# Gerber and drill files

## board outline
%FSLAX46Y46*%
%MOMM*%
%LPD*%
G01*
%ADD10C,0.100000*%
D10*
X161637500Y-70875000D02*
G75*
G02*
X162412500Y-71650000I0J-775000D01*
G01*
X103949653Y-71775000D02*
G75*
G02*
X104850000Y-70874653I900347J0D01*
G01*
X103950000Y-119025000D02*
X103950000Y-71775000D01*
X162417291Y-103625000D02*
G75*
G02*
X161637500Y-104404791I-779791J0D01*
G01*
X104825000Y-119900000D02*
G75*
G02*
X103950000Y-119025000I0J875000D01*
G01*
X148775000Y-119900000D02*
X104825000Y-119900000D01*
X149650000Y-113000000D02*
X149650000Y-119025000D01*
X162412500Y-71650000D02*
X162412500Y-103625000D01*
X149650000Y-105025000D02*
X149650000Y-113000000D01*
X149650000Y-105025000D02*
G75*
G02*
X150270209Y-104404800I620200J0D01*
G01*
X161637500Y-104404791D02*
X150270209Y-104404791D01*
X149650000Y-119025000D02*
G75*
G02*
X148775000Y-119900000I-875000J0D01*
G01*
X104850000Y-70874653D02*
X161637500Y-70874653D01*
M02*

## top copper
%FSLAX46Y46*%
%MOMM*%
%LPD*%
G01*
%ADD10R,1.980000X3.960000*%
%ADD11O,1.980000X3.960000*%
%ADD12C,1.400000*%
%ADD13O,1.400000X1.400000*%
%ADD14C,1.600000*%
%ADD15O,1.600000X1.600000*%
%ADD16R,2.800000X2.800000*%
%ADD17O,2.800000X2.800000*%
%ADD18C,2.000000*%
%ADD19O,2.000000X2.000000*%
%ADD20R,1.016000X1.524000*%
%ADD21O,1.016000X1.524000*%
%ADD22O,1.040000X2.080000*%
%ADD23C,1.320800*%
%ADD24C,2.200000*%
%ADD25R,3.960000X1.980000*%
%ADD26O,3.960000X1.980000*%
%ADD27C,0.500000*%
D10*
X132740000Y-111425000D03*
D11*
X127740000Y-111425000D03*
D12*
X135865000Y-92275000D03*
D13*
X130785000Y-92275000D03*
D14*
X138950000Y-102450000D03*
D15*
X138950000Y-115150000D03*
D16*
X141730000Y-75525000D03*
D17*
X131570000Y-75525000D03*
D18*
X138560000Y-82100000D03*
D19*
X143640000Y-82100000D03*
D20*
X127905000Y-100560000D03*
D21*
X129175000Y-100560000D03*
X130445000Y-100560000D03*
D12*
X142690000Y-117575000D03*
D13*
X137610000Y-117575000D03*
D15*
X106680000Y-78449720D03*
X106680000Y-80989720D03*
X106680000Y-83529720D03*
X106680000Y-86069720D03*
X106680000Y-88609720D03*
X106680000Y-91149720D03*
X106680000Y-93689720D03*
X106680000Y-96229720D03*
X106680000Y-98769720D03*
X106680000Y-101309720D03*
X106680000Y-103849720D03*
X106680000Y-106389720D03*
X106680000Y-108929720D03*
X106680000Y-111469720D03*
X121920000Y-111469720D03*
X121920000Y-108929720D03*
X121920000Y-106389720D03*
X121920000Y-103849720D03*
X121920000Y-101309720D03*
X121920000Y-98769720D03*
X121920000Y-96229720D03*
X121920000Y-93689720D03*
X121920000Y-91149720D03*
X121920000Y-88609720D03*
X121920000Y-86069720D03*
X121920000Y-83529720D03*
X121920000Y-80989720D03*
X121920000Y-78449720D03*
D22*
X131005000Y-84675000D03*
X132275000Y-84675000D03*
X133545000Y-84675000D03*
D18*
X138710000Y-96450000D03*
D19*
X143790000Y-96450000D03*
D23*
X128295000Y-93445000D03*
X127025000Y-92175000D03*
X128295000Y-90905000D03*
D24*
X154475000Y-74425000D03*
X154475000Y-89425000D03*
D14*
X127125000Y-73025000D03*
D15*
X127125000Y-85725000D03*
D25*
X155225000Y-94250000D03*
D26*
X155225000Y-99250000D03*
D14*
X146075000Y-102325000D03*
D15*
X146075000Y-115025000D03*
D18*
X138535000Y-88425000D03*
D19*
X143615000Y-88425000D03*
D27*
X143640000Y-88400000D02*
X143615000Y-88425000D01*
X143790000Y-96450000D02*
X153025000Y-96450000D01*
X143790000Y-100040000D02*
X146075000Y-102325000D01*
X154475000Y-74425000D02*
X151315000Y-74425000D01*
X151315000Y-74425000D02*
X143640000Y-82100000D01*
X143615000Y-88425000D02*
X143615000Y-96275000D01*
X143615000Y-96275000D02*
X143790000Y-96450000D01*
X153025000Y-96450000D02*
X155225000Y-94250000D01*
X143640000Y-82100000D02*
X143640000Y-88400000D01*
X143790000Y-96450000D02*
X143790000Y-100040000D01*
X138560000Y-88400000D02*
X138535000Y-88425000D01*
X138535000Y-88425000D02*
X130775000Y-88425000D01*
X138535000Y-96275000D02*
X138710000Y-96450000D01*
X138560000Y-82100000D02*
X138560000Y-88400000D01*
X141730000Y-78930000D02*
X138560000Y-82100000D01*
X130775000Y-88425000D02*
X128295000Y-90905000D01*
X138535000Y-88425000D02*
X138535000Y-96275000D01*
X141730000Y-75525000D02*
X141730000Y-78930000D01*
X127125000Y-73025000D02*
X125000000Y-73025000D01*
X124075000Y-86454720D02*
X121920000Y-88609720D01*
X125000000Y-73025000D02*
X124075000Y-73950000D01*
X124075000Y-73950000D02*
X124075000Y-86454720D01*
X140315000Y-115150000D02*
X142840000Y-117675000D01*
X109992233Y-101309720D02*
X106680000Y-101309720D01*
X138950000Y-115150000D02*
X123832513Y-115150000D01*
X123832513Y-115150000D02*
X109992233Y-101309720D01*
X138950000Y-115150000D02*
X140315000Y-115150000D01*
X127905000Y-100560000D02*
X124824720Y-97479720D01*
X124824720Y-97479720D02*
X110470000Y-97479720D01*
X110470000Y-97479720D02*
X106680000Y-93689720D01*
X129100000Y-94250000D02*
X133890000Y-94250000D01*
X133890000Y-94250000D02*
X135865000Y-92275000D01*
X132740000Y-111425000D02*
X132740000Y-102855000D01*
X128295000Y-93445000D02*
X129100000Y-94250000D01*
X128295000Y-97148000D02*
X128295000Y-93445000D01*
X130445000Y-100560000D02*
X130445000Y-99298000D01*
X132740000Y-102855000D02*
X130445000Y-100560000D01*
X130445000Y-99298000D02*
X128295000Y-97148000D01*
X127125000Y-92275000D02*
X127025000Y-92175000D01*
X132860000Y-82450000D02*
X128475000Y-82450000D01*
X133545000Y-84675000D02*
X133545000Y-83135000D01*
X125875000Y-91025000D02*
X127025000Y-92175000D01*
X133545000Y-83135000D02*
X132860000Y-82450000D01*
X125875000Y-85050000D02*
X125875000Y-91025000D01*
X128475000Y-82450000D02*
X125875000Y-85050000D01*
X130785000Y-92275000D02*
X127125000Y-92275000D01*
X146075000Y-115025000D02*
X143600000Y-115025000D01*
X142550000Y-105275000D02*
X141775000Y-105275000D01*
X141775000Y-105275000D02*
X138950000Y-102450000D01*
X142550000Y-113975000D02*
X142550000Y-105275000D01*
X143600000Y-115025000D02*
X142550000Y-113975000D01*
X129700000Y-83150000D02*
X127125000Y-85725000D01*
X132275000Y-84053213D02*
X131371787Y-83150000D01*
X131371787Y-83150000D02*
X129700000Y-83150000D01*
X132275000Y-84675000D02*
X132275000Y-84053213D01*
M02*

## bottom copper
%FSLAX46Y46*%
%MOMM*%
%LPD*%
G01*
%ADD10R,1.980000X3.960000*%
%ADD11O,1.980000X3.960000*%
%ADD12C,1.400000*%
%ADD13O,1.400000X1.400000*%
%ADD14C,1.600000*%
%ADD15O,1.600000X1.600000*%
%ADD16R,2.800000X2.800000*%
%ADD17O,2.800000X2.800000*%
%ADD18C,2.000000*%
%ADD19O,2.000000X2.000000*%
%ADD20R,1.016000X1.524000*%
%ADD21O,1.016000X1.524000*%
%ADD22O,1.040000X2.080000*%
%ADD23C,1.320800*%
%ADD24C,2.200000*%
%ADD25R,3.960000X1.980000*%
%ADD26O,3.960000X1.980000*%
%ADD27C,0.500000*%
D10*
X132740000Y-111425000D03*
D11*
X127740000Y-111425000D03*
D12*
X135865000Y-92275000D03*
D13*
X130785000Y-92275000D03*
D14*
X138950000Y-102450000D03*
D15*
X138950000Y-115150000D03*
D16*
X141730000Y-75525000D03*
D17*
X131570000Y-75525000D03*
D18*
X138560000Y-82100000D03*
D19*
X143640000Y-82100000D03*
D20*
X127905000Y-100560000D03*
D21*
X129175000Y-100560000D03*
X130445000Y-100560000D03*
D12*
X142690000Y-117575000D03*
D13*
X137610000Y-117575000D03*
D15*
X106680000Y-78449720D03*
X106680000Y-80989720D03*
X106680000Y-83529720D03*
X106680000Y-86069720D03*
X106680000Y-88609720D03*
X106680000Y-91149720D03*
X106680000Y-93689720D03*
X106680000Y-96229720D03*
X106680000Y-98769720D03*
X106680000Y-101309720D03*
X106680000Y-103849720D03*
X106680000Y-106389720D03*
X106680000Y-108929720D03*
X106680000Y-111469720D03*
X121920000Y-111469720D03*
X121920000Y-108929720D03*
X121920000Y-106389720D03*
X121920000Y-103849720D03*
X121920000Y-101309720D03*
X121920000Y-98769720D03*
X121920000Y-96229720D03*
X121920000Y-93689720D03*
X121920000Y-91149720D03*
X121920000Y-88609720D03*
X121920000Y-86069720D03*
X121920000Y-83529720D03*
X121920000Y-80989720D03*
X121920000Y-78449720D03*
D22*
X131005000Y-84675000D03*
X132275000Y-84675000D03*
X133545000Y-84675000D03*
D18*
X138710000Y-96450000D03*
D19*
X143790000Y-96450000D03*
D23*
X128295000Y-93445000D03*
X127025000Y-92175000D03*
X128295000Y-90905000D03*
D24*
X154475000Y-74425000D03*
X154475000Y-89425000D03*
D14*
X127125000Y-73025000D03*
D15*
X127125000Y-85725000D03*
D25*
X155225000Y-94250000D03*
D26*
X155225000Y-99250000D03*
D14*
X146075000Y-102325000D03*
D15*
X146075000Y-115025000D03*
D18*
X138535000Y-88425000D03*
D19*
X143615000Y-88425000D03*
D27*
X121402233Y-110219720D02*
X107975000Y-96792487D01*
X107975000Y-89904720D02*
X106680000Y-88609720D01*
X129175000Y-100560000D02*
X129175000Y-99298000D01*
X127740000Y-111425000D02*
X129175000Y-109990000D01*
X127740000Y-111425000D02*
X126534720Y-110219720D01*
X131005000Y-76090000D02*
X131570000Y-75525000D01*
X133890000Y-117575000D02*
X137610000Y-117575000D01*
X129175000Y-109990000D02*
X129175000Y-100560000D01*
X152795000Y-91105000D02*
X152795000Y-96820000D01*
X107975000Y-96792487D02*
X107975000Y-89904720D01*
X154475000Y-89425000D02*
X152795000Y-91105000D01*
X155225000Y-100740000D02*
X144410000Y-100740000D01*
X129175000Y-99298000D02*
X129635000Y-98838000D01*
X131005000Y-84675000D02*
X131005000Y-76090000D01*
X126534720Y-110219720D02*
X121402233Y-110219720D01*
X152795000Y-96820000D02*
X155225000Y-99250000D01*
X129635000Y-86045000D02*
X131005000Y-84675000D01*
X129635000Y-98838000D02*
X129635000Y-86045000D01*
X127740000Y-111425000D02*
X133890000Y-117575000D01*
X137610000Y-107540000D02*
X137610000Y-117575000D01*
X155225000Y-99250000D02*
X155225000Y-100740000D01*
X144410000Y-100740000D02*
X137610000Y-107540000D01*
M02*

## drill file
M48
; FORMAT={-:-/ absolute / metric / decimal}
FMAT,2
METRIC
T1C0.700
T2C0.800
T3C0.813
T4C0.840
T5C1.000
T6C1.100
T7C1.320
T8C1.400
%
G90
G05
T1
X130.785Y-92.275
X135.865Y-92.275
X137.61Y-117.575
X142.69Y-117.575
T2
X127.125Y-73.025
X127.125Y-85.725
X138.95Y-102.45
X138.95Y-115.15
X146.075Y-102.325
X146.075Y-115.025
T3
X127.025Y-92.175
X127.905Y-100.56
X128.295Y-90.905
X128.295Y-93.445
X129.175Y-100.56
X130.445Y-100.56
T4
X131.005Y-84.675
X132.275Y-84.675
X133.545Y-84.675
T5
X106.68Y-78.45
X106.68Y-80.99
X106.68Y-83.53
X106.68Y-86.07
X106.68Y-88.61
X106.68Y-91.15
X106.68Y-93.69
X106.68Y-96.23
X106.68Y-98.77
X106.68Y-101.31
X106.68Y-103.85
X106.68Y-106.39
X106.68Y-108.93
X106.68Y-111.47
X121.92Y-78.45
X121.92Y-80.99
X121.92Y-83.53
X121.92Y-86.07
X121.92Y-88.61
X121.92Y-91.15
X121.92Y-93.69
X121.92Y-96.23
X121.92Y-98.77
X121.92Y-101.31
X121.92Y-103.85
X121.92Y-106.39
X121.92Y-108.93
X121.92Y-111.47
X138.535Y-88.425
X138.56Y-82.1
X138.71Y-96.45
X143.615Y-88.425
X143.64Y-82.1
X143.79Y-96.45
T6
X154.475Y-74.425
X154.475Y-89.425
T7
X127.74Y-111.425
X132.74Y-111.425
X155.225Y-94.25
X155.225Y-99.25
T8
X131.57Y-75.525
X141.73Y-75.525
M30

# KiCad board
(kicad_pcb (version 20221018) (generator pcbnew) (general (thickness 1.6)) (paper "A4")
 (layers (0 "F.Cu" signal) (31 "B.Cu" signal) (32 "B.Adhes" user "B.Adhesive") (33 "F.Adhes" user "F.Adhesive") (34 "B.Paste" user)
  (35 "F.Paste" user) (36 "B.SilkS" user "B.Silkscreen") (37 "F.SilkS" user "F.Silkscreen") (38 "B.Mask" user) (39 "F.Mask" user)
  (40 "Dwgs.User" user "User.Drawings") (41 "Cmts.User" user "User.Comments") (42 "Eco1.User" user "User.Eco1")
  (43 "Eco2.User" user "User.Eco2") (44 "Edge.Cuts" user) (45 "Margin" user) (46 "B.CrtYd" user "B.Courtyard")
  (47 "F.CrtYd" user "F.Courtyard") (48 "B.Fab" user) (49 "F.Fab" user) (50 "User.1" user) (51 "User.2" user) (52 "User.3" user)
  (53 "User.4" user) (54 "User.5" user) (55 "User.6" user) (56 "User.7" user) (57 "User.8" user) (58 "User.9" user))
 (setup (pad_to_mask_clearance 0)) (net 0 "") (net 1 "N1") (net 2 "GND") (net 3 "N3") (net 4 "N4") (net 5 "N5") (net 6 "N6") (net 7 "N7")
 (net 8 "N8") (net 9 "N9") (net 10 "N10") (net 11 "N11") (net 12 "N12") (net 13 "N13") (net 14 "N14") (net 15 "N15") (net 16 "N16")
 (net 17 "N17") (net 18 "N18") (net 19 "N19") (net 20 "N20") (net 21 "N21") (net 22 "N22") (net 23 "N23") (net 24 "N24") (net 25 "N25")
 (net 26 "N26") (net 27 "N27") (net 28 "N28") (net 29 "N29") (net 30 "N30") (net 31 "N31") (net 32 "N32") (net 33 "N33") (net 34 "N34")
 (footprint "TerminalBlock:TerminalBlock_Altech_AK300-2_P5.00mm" (layer "F.Cu") (at 132.74 111.425 180)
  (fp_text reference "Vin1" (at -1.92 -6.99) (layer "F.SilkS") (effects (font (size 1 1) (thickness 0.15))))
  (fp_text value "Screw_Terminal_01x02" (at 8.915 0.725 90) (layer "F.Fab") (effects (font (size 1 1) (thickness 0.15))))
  (pad "1" thru_hole rect (at 0 0 180) (size 1.98 3.96) (drill 1.32) (layers "*.Cu" "*.Mask") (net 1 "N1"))
  (pad "2" thru_hole oval (at 5 0 180) (size 1.98 3.96) (drill 1.32) (layers "*.Cu" "*.Mask") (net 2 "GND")))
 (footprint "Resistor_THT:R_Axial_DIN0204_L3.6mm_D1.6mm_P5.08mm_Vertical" (layer "F.Cu") (at 135.865 92.275 180)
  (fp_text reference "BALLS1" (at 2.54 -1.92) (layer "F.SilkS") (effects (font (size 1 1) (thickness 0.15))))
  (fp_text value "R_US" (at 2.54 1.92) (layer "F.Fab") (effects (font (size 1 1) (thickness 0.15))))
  (pad "1" thru_hole circle (at 0 0 180) (size 1.4 1.4) (drill 0.7) (layers "*.Cu" "*.Mask") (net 1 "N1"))
  (pad "2" thru_hole oval (at 5.08 0 180) (size 1.4 1.4) (drill 0.7) (layers "*.Cu" "*.Mask") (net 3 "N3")))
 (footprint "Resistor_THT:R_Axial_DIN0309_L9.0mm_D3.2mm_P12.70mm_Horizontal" (layer "F.Cu") (at 138.95 102.45 -90)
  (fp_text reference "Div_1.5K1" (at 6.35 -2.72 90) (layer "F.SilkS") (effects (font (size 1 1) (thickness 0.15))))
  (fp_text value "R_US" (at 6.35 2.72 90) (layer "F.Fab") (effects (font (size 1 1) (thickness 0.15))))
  (pad "1" thru_hole circle (at 0 0 270) (size 1.6 1.6) (drill 0.8) (layers "*.Cu" "*.Mask") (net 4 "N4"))
  (pad "2" thru_hole oval (at 12.7 0 270) (size 1.6 1.6) (drill 0.8) (layers "*.Cu" "*.Mask") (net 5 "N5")))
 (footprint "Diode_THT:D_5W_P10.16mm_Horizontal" (layer "F.Cu") (at 141.73 75.525 180)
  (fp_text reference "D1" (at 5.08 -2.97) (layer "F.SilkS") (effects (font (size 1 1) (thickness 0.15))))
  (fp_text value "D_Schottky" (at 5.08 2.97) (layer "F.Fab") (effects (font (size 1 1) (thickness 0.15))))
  (pad "1" thru_hole rect (at 0 0 180) (size 2.8 2.8) (drill 1.4) (layers "*.Cu" "*.Mask") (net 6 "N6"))
  (pad "2" thru_hole oval (at 10.16 0 180) (size 2.8 2.8) (drill 1.4) (layers "*.Cu" "*.Mask") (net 2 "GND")))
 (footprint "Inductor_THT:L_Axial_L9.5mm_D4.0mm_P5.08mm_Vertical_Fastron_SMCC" (layer "F.Cu") (at 138.56 82.1)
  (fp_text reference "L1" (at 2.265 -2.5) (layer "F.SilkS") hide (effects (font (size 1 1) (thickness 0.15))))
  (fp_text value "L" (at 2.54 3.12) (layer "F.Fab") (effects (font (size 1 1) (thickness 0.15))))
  (pad "1" thru_hole circle (at 0 0) (size 2 2) (drill 1) (layers "*.Cu" "*.Mask") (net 6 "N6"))
  (pad "2" thru_hole oval (at 5.08 0) (size 2 2) (drill 1) (layers "*.Cu" "*.Mask") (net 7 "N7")))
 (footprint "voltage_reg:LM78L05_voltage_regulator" (layer "F.Cu") (at 127.905 100.56)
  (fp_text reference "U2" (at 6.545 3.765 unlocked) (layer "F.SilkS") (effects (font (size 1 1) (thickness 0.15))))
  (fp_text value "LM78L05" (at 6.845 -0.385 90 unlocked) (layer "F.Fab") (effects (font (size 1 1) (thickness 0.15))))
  (pad "1" thru_hole rect (at 0 0) (size 1.016 1.524) (drill 0.8128) (layers "*.Cu" "*.Mask") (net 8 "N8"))
  (pad "2" thru_hole oval (at 1.27 0) (size 1.016 1.524) (drill 0.8128) (layers "*.Cu" "*.Mask") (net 2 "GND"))
  (pad "3" thru_hole oval (at 2.54 0) (size 1.016 1.524) (drill 0.8128) (layers "*.Cu" "*.Mask") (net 1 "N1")))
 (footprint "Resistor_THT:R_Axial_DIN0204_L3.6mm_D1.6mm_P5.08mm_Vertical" (layer "F.Cu") (at 142.69 117.575 180)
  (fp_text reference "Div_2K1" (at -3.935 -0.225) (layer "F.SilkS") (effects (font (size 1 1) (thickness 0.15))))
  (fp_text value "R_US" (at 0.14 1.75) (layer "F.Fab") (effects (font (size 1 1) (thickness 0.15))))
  (pad "1" thru_hole circle (at 0 0 180) (size 1.4 1.4) (drill 0.7) (layers "*.Cu" "*.Mask") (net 5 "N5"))
  (pad "2" thru_hole oval (at 5.08 0 180) (size 1.4 1.4) (drill 0.7) (layers "*.Cu" "*.Mask") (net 2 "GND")))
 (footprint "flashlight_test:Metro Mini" (layer "F.Cu") (at 114.3508 94.85812)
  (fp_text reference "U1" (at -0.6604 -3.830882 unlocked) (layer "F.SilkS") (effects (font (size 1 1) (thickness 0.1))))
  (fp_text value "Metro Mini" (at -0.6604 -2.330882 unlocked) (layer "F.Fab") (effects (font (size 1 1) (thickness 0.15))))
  (pad "1" thru_hole oval (at -7.6708 -16.4084 180) (size 1.6 1.6) (drill 1) (layers "*.Cu" "*.Mask") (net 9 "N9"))
  (pad "2" thru_hole oval (at -7.6708 -13.8684 180) (size 1.6 1.6) (drill 1) (layers "*.Cu" "*.Mask") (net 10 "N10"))
  (pad "3" thru_hole oval (at -7.6708 -11.3284 180) (size 1.6 1.6) (drill 1) (layers "*.Cu" "*.Mask") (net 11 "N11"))
  (pad "4" thru_hole oval (at -7.6708 -8.7884 180) (size 1.6 1.6) (drill 1) (layers "*.Cu" "*.Mask") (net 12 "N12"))
  (pad "5" thru_hole oval (at -7.6708 -6.2484 180) (size 1.6 1.6) (drill 1) (layers "*.Cu" "*.Mask") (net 2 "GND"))
  (pad "6" thru_hole oval (at -7.6708 -3.7084 180) (size 1.6 1.6) (drill 1) (layers "*.Cu" "*.Mask") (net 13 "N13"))
  (pad "7" thru_hole oval (at -7.6708 -1.1684 180) (size 1.6 1.6) (drill 1) (layers "*.Cu" "*.Mask") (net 8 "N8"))
  (pad "8" thru_hole oval (at -7.6708 1.3716 180) (size 1.6 1.6) (drill 1) (layers "*.Cu" "*.Mask") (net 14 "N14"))
  (pad "9" thru_hole oval (at -7.6708 3.9116 180) (size 1.6 1.6) (drill 1) (layers "*.Cu" "*.Mask") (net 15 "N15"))
  (pad "10" thru_hole oval (at -7.6708 6.4516 180) (size 1.6 1.6) (drill 1) (layers "*.Cu" "*.Mask") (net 5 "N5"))
  (pad "11" thru_hole oval (at -7.6708 8.9916 180) (size 1.6 1.6) (drill 1) (layers "*.Cu" "*.Mask") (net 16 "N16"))
  (pad "12" thru_hole oval (at -7.6708 11.5316 180) (size 1.6 1.6) (drill 1) (layers "*.Cu" "*.Mask") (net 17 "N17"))
  (pad "13" thru_hole oval (at -7.6708 14.0716 180) (size 1.6 1.6) (drill 1) (layers "*.Cu" "*.Mask") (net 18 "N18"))
  (pad "14" thru_hole oval (at -7.6708 16.6116 180) (size 1.6 1.6) (drill 1) (layers "*.Cu" "*.Mask") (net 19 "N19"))
  (pad "15" thru_hole oval (at 7.5692 16.6116 180) (size 1.6 1.6) (drill 1) (layers "*.Cu" "*.Mask") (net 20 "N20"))
  (pad "16" thru_hole oval (at 7.5692 14.0716 180) (size 1.6 1.6) (drill 1) (layers "*.Cu" "*.Mask") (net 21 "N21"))
  (pad "17" thru_hole oval (at 7.5692 11.5316 180) (size 1.6 1.6) (drill 1) (layers "*.Cu" "*.Mask") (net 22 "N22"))
  (pad "18" thru_hole oval (at 7.5692 8.9916 180) (size 1.6 1.6) (drill 1) (layers "*.Cu" "*.Mask") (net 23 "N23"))
  (pad "19" thru_hole oval (at 7.5692 6.4516 180) (size 1.6 1.6) (drill 1) (layers "*.Cu" "*.Mask") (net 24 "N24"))
  (pad "20" thru_hole oval (at 7.5692 3.9116 180) (size 1.6 1.6) (drill 1) (layers "*.Cu" "*.Mask") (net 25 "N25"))
  (pad "21" thru_hole oval (at 7.5692 1.3716 180) (size 1.6 1.6) (drill 1) (layers "*.Cu" "*.Mask") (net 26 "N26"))
  (pad "22" thru_hole oval (at 7.5692 -1.1684 180) (size 1.6 1.6) (drill 1) (layers "*.Cu" "*.Mask") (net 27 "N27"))
  (pad "23" thru_hole oval (at 7.5692 -3.7084 180) (size 1.6 1.6) (drill 1) (layers "*.Cu" "*.Mask") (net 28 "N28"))
  (pad "24" thru_hole oval (at 7.5692 -6.2484 180) (size 1.6 1.6) (drill 1) (layers "*.Cu" "*.Mask") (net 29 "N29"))
  (pad "25" thru_hole oval (at 7.5692 -8.7884 180) (size 1.6 1.6) (drill 1) (layers "*.Cu" "*.Mask") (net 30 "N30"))
  (pad "26" thru_hole oval (at 7.5692 -11.3284 180) (size 1.6 1.6) (drill 1) (layers "*.Cu" "*.Mask") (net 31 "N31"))
  (pad "27" thru_hole oval (at 7.5692 -13.8684 180) (size 1.6 1.6) (drill 1) (layers "*.Cu" "*.Mask") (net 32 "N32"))
  (pad "28" thru_hole oval (at 7.5692 -16.4084 180) (size 1.6 1.6) (drill 1) (layers "*.Cu" "*.Mask") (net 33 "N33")))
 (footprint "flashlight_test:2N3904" (layer "F.Cu") (at 132.275 84.675)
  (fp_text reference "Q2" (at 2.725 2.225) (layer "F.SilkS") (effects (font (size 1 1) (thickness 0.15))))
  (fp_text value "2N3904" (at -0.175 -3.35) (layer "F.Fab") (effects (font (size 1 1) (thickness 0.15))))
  (pad "1" thru_hole oval (at -1.27 0) (size 1.04 2.08) (drill 0.84) (layers "*.Cu" "*.Mask") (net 2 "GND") (solder_mask_margin 0.102))
  (pad "2" thru_hole oval (at 0 0) (size 1.04 2.08) (drill 0.84) (layers "*.Cu" "*.Mask") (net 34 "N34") (solder_mask_margin 0.102))
  (pad "3" thru_hole oval (at 1.27 0) (size 1.04 2.08) (drill 0.84) (layers "*.Cu" "*.Mask") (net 3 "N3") (solder_mask_margin 0.102)))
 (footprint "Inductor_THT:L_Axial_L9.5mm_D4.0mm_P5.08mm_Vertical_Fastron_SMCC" (layer "F.Cu") (at 138.71 96.45)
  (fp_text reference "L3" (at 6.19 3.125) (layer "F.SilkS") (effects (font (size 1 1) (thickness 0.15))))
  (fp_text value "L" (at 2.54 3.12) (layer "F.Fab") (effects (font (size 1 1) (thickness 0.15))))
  (pad "1" thru_hole circle (at 0 0) (size 2 2) (drill 1) (layers "*.Cu" "*.Mask") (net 6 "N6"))
  (pad "2" thru_hole oval (at 5.08 0) (size 2 2) (drill 1) (layers "*.Cu" "*.Mask") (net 7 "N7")))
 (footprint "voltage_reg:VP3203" (layer "F.Cu") (at 128.295 93.445 90)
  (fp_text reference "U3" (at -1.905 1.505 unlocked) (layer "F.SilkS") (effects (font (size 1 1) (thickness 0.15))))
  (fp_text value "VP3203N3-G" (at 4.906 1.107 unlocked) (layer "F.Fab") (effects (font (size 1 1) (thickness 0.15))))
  (pad "1" thru_hole circle (at 0 0 90) (size 1.3208 1.3208) (drill 0.8128) (layers "*.Cu" "*.Mask") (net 1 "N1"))
  (pad "2" thru_hole circle (at 1.27 -1.27 90) (size 1.3208 1.3208) (drill 0.8128) (layers "*.Cu" "*.Mask") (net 3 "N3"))
  (pad "3" thru_hole circle (at 2.54 0 90) (size 1.3208 1.3208) (drill 0.8128) (layers "*.Cu" "*.Mask") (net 6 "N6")))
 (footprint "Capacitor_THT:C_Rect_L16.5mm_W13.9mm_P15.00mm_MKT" (layer "F.Cu") (at 154.475 74.425 -90)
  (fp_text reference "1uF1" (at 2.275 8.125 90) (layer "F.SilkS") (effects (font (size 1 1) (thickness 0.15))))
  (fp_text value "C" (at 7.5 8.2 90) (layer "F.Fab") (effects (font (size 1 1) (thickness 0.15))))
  (pad "1" thru_hole circle (at 0 0 270) (size 2.2 2.2) (drill 1.1) (layers "*.Cu" "*.Mask") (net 7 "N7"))
  (pad "2" thru_hole circle (at 15 0 270) (size 2.2 2.2) (drill 1.1) (layers "*.Cu" "*.Mask") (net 2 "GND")))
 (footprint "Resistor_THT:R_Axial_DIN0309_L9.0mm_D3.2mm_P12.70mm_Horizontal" (layer "F.Cu") (at 127.125 73.025 -90)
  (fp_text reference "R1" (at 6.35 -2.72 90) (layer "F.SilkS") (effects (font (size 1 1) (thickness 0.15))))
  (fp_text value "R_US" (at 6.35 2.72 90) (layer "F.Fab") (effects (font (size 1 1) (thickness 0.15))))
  (pad "1" thru_hole circle (at 0 0 270) (size 1.6 1.6) (drill 0.8) (layers "*.Cu" "*.Mask") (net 29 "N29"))
  (pad "2" thru_hole oval (at 12.7 0 270) (size 1.6 1.6) (drill 0.8) (layers "*.Cu" "*.Mask") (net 34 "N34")))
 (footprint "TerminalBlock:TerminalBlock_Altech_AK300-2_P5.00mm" (layer "F.Cu") (at 155.225 94.25 -90)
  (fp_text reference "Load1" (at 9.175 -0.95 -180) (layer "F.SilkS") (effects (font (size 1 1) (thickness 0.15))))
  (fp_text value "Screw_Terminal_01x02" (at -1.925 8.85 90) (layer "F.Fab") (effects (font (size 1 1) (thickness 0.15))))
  (pad "1" thru_hole rect (at 0 0 270) (size 1.98 3.96) (drill 1.32) (layers "*.Cu" "*.Mask") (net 7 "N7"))
  (pad "2" thru_hole oval (at 5 0 270) (size 1.98 3.96) (drill 1.32) (layers "*.Cu" "*.Mask") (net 2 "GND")))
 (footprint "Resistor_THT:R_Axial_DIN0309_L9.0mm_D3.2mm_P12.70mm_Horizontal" (layer "F.Cu") (at 146.075 102.325 -90)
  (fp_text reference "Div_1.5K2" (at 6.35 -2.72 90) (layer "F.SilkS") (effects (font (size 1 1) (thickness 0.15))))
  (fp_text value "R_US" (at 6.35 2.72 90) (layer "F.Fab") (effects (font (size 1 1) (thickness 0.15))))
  (pad "1" thru_hole circle (at 0 0 270) (size 1.6 1.6) (drill 0.8) (layers "*.Cu" "*.Mask") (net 7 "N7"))
  (pad "2" thru_hole oval (at 12.7 0 270) (size 1.6 1.6) (drill 0.8) (layers "*.Cu" "*.Mask") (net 4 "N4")))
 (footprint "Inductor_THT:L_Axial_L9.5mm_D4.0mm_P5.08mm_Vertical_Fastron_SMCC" (layer "F.Cu") (at 138.535 88.425)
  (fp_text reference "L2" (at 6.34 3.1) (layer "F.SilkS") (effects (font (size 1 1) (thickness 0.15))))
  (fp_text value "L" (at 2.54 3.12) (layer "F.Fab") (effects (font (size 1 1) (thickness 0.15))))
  (pad "1" thru_hole circle (at 0 0) (size 2 2) (drill 1) (layers "*.Cu" "*.Mask") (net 6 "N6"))
  (pad "2" thru_hole oval (at 5.08 0) (size 2 2) (drill 1) (layers "*.Cu" "*.Mask") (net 7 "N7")))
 (gr_arc (start 161.6375 70.875) (mid 162.185507 71.101992) (end 162.4125 71.65) (stroke (width 0.1) (type default)) (layer "Edge.Cuts"))
 (gr_arc (start 103.949653 71.775) (mid 104.213359 71.138359) (end 104.85 70.874653) (stroke (width 0.1) (type default)) (layer "Edge.Cuts"))
 (gr_line (start 103.95 119.025) (end 103.95 71.775) (stroke (width 0.1) (type default)) (layer "Edge.Cuts"))
 (gr_arc (start 162.417291 103.625) (mid 162.188895 104.176395) (end 161.6375 104.404791) (stroke (width 0.1) (type default))
  (layer "Edge.Cuts"))
 (gr_arc (start 104.825 119.9) (mid 104.206282 119.643718) (end 103.95 119.025) (stroke (width 0.1) (type default)) (layer "Edge.Cuts"))
 (gr_line (start 148.775 119.9) (end 104.825 119.9) (stroke (width 0.1) (type default)) (layer "Edge.Cuts"))
 (gr_line (start 149.65 113) (end 149.65 119.025) (stroke (width 0.1) (type default)) (layer "Edge.Cuts"))
 (gr_line (start 162.4125 71.65) (end 162.4125 103.625) (stroke (width 0.1) (type default)) (layer "Edge.Cuts"))
 (gr_line (start 149.65 105.025) (end 149.65 113) (stroke (width 0.1) (type default)) (layer "Edge.Cuts"))
 (gr_arc (start 149.65 105.025) (mid 149.831655 104.586446) (end 150.270209 104.404791) (stroke (width 0.1) (type default))
  (layer "Edge.Cuts"))
 (gr_line (start 161.6375 104.404791) (end 150.270209 104.404791) (stroke (width 0.1) (type default)) (layer "Edge.Cuts"))
 (gr_arc (start 149.65 119.025) (mid 149.393718 119.643718) (end 148.775 119.9) (stroke (width 0.1) (type default)) (layer "Edge.Cuts"))
 (gr_line (start 104.85 70.874653) (end 161.6375 70.874653) (stroke (width 0.1) (type default)) (layer "Edge.Cuts"))
 (segment (start 143.64 88.4) (end 143.615 88.425) (width 0.5) (layer "F.Cu") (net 7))
 (segment (start 143.79 96.45) (end 153.025 96.45) (width 0.5) (layer "F.Cu") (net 7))
 (segment (start 143.79 100.04) (end 146.075 102.325) (width 0.5) (layer "F.Cu") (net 7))
 (segment (start 154.475 74.425) (end 151.315 74.425) (width 0.5) (layer "F.Cu") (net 7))
 (segment (start 151.315 74.425) (end 143.64 82.1) (width 0.5) (layer "F.Cu") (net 7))
 (segment (start 143.615 88.425) (end 143.615 96.275) (width 0.5) (layer "F.Cu") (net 7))
 (segment (start 143.615 96.275) (end 143.79 96.45) (width 0.5) (layer "F.Cu") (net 7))
 (segment (start 153.025 96.45) (end 155.225 94.25) (width 0.5) (layer "F.Cu") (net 7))
 (segment (start 143.64 82.1) (end 143.64 88.4) (width 0.5) (layer "F.Cu") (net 7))
 (segment (start 143.79 96.45) (end 143.79 100.04) (width 0.5) (layer "F.Cu") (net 7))
 (segment (start 138.56 88.4) (end 138.535 88.425) (width 0.5) (layer "F.Cu") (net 6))
 (segment (start 138.535 88.425) (end 130.775 88.425) (width 0.5) (layer "F.Cu") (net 6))
 (segment (start 138.535 96.275) (end 138.71 96.45) (width 0.5) (layer "F.Cu") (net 6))
 (segment (start 138.56 82.1) (end 138.56 88.4) (width 0.5) (layer "F.Cu") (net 6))
 (segment (start 141.73 78.93) (end 138.56 82.1) (width 0.5) (layer "F.Cu") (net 6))
 (segment (start 130.775 88.425) (end 128.295 90.905) (width 0.5) (layer "F.Cu") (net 6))
 (segment (start 138.535 88.425) (end 138.535 96.275) (width 0.5) (layer "F.Cu") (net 6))
 (segment (start 141.73 75.525) (end 141.73 78.93) (width 0.5) (layer "F.Cu") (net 6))
 (segment (start 121.402233 110.21972) (end 107.975 96.792487) (width 0.5) (layer "B.Cu") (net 2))
 (segment (start 107.975 89.90472) (end 106.68 88.60972) (width 0.5) (layer "B.Cu") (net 2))
 (segment (start 129.175 100.56) (end 129.175 99.298) (width 0.5) (layer "B.Cu") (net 2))
 (segment (start 127.74 111.425) (end 129.175 109.99) (width 0.5) (layer "B.Cu") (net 2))
 (segment (start 127.74 111.425) (end 126.53472 110.21972) (width 0.5) (layer "B.Cu") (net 2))
 (segment (start 131.005 76.09) (end 131.57 75.525) (width 0.5) (layer "B.Cu") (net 2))
 (segment (start 133.89 117.575) (end 137.61 117.575) (width 0.5) (layer "B.Cu") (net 2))
 (segment (start 129.175 109.99) (end 129.175 100.56) (width 0.5) (layer "B.Cu") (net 2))
 (segment (start 152.795 91.105) (end 152.795 96.82) (width 0.5) (layer "B.Cu") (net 2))
 (segment (start 107.975 96.792487) (end 107.975 89.90472) (width 0.5) (layer "B.Cu") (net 2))
 (segment (start 154.475 89.425) (end 152.795 91.105) (width 0.5) (layer "B.Cu") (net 2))
 (segment (start 155.225 100.74) (end 144.41 100.74) (width 0.5) (layer "B.Cu") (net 2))
 (segment (start 129.175 99.298) (end 129.635 98.838) (width 0.5) (layer "B.Cu") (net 2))
 (segment (start 131.005 84.675) (end 131.005 76.09) (width 0.5) (layer "B.Cu") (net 2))
 (segment (start 126.53472 110.21972) (end 121.402233 110.21972) (width 0.5) (layer "B.Cu") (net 2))
 (segment (start 152.795 96.82) (end 155.225 99.25) (width 0.5) (layer "B.Cu") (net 2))
 (segment (start 129.635 86.045) (end 131.005 84.675) (width 0.5) (layer "B.Cu") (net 2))
 (segment (start 129.635 98.838) (end 129.635 86.045) (width 0.5) (layer "B.Cu") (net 2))
 (segment (start 127.74 111.425) (end 133.89 117.575) (width 0.5) (layer "B.Cu") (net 2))
 (segment (start 137.61 107.54) (end 137.61 117.575) (width 0.5) (layer "B.Cu") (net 2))
 (segment (start 155.225 99.25) (end 155.225 100.74) (width 0.5) (layer "B.Cu") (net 2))
 (segment (start 144.41 100.74) (end 137.61 107.54) (width 0.5) (layer "B.Cu") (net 2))
 (segment (start 127.125 73.025) (end 125 73.025) (width 0.5) (layer "F.Cu") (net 29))
 (segment (start 124.075 86.45472) (end 121.92 88.60972) (width 0.5) (layer "F.Cu") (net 29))
 (segment (start 125 73.025) (end 124.075 73.95) (width 0.5) (layer "F.Cu") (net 29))
 (segment (start 124.075 73.95) (end 124.075 86.45472) (width 0.5) (layer "F.Cu") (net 29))
 (segment (start 140.315 115.15) (end 142.84 117.675) (width 0.5) (layer "F.Cu") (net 5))
 (segment (start 109.992233 101.30972) (end 106.68 101.30972) (width 0.5) (layer "F.Cu") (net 5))
 (segment (start 138.95 115.15) (end 123.832513 115.15) (width 0.5) (layer "F.Cu") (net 5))
 (segment (start 123.832513 115.15) (end 109.992233 101.30972) (width 0.5) (layer "F.Cu") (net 5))
 (segment (start 138.95 115.15) (end 140.315 115.15) (width 0.5) (layer "F.Cu") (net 5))
 (segment (start 127.905 100.56) (end 124.82472 97.47972) (width 0.5) (layer "F.Cu") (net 8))
 (segment (start 124.82472 97.47972) (end 110.47 97.47972) (width 0.5) (layer "F.Cu") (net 8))
 (segment (start 110.47 97.47972) (end 106.68 93.68972) (width 0.5) (layer "F.Cu") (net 8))
 (segment (start 129.1 94.25) (end 133.89 94.25) (width 0.5) (layer "F.Cu") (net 1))
 (segment (start 133.89 94.25) (end 135.865 92.275) (width 0.5) (layer "F.Cu") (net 1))
 (segment (start 132.74 111.425) (end 132.74 102.855) (width 0.5) (layer "F.Cu") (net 1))
 (segment (start 128.295 93.445) (end 129.1 94.25) (width 0.5) (layer "F.Cu") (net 1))
 (segment (start 128.295 97.148) (end 128.295 93.445) (width 0.5) (layer "F.Cu") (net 1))
 (segment (start 130.445 100.56) (end 130.445 99.298) (width 0.5) (layer "F.Cu") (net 1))
 (segment (start 132.74 102.855) (end 130.445 100.56) (width 0.5) (layer "F.Cu") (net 1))
 (segment (start 130.445 99.298) (end 128.295 97.148) (width 0.5) (layer "F.Cu") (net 1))
 (segment (start 127.125 92.275) (end 127.025 92.175) (width 0.5) (layer "F.Cu") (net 3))
 (segment (start 132.86 82.45) (end 128.475 82.45) (width 0.5) (layer "F.Cu") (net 3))
 (segment (start 133.545 84.675) (end 133.545 83.135) (width 0.5) (layer "F.Cu") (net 3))
 (segment (start 125.875 91.025) (end 127.025 92.175) (width 0.5) (layer "F.Cu") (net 3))
 (segment (start 133.545 83.135) (end 132.86 82.45) (width 0.5) (layer "F.Cu") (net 3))
 (segment (start 125.875 85.05) (end 125.875 91.025) (width 0.5) (layer "F.Cu") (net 3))
 (segment (start 128.475 82.45) (end 125.875 85.05) (width 0.5) (layer "F.Cu") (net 3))
 (segment (start 130.785 92.275) (end 127.125 92.275) (width 0.5) (layer "F.Cu") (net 3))
 (segment (start 146.075 115.025) (end 143.6 115.025) (width 0.5) (layer "F.Cu") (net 4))
 (segment (start 142.55 105.275) (end 141.775 105.275) (width 0.5) (layer "F.Cu") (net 4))
 (segment (start 141.775 105.275) (end 138.95 102.45) (width 0.5) (layer "F.Cu") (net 4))
 (segment (start 142.55 113.975) (end 142.55 105.275) (width 0.5) (layer "F.Cu") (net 4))
 (segment (start 143.6 115.025) (end 142.55 113.975) (width 0.5) (layer "F.Cu") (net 4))
 (segment (start 129.7 83.15) (end 127.125 85.725) (width 0.5) (layer "F.Cu") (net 34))
 (segment (start 132.275 84.053213) (end 131.371787 83.15) (width 0.5) (layer "F.Cu") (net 34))
 (segment (start 131.371787 83.15) (end 129.7 83.15) (width 0.5) (layer "F.Cu") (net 34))
 (segment (start 132.275 84.675) (end 132.275 84.053213) (width 0.5) (layer "F.Cu") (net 34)))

